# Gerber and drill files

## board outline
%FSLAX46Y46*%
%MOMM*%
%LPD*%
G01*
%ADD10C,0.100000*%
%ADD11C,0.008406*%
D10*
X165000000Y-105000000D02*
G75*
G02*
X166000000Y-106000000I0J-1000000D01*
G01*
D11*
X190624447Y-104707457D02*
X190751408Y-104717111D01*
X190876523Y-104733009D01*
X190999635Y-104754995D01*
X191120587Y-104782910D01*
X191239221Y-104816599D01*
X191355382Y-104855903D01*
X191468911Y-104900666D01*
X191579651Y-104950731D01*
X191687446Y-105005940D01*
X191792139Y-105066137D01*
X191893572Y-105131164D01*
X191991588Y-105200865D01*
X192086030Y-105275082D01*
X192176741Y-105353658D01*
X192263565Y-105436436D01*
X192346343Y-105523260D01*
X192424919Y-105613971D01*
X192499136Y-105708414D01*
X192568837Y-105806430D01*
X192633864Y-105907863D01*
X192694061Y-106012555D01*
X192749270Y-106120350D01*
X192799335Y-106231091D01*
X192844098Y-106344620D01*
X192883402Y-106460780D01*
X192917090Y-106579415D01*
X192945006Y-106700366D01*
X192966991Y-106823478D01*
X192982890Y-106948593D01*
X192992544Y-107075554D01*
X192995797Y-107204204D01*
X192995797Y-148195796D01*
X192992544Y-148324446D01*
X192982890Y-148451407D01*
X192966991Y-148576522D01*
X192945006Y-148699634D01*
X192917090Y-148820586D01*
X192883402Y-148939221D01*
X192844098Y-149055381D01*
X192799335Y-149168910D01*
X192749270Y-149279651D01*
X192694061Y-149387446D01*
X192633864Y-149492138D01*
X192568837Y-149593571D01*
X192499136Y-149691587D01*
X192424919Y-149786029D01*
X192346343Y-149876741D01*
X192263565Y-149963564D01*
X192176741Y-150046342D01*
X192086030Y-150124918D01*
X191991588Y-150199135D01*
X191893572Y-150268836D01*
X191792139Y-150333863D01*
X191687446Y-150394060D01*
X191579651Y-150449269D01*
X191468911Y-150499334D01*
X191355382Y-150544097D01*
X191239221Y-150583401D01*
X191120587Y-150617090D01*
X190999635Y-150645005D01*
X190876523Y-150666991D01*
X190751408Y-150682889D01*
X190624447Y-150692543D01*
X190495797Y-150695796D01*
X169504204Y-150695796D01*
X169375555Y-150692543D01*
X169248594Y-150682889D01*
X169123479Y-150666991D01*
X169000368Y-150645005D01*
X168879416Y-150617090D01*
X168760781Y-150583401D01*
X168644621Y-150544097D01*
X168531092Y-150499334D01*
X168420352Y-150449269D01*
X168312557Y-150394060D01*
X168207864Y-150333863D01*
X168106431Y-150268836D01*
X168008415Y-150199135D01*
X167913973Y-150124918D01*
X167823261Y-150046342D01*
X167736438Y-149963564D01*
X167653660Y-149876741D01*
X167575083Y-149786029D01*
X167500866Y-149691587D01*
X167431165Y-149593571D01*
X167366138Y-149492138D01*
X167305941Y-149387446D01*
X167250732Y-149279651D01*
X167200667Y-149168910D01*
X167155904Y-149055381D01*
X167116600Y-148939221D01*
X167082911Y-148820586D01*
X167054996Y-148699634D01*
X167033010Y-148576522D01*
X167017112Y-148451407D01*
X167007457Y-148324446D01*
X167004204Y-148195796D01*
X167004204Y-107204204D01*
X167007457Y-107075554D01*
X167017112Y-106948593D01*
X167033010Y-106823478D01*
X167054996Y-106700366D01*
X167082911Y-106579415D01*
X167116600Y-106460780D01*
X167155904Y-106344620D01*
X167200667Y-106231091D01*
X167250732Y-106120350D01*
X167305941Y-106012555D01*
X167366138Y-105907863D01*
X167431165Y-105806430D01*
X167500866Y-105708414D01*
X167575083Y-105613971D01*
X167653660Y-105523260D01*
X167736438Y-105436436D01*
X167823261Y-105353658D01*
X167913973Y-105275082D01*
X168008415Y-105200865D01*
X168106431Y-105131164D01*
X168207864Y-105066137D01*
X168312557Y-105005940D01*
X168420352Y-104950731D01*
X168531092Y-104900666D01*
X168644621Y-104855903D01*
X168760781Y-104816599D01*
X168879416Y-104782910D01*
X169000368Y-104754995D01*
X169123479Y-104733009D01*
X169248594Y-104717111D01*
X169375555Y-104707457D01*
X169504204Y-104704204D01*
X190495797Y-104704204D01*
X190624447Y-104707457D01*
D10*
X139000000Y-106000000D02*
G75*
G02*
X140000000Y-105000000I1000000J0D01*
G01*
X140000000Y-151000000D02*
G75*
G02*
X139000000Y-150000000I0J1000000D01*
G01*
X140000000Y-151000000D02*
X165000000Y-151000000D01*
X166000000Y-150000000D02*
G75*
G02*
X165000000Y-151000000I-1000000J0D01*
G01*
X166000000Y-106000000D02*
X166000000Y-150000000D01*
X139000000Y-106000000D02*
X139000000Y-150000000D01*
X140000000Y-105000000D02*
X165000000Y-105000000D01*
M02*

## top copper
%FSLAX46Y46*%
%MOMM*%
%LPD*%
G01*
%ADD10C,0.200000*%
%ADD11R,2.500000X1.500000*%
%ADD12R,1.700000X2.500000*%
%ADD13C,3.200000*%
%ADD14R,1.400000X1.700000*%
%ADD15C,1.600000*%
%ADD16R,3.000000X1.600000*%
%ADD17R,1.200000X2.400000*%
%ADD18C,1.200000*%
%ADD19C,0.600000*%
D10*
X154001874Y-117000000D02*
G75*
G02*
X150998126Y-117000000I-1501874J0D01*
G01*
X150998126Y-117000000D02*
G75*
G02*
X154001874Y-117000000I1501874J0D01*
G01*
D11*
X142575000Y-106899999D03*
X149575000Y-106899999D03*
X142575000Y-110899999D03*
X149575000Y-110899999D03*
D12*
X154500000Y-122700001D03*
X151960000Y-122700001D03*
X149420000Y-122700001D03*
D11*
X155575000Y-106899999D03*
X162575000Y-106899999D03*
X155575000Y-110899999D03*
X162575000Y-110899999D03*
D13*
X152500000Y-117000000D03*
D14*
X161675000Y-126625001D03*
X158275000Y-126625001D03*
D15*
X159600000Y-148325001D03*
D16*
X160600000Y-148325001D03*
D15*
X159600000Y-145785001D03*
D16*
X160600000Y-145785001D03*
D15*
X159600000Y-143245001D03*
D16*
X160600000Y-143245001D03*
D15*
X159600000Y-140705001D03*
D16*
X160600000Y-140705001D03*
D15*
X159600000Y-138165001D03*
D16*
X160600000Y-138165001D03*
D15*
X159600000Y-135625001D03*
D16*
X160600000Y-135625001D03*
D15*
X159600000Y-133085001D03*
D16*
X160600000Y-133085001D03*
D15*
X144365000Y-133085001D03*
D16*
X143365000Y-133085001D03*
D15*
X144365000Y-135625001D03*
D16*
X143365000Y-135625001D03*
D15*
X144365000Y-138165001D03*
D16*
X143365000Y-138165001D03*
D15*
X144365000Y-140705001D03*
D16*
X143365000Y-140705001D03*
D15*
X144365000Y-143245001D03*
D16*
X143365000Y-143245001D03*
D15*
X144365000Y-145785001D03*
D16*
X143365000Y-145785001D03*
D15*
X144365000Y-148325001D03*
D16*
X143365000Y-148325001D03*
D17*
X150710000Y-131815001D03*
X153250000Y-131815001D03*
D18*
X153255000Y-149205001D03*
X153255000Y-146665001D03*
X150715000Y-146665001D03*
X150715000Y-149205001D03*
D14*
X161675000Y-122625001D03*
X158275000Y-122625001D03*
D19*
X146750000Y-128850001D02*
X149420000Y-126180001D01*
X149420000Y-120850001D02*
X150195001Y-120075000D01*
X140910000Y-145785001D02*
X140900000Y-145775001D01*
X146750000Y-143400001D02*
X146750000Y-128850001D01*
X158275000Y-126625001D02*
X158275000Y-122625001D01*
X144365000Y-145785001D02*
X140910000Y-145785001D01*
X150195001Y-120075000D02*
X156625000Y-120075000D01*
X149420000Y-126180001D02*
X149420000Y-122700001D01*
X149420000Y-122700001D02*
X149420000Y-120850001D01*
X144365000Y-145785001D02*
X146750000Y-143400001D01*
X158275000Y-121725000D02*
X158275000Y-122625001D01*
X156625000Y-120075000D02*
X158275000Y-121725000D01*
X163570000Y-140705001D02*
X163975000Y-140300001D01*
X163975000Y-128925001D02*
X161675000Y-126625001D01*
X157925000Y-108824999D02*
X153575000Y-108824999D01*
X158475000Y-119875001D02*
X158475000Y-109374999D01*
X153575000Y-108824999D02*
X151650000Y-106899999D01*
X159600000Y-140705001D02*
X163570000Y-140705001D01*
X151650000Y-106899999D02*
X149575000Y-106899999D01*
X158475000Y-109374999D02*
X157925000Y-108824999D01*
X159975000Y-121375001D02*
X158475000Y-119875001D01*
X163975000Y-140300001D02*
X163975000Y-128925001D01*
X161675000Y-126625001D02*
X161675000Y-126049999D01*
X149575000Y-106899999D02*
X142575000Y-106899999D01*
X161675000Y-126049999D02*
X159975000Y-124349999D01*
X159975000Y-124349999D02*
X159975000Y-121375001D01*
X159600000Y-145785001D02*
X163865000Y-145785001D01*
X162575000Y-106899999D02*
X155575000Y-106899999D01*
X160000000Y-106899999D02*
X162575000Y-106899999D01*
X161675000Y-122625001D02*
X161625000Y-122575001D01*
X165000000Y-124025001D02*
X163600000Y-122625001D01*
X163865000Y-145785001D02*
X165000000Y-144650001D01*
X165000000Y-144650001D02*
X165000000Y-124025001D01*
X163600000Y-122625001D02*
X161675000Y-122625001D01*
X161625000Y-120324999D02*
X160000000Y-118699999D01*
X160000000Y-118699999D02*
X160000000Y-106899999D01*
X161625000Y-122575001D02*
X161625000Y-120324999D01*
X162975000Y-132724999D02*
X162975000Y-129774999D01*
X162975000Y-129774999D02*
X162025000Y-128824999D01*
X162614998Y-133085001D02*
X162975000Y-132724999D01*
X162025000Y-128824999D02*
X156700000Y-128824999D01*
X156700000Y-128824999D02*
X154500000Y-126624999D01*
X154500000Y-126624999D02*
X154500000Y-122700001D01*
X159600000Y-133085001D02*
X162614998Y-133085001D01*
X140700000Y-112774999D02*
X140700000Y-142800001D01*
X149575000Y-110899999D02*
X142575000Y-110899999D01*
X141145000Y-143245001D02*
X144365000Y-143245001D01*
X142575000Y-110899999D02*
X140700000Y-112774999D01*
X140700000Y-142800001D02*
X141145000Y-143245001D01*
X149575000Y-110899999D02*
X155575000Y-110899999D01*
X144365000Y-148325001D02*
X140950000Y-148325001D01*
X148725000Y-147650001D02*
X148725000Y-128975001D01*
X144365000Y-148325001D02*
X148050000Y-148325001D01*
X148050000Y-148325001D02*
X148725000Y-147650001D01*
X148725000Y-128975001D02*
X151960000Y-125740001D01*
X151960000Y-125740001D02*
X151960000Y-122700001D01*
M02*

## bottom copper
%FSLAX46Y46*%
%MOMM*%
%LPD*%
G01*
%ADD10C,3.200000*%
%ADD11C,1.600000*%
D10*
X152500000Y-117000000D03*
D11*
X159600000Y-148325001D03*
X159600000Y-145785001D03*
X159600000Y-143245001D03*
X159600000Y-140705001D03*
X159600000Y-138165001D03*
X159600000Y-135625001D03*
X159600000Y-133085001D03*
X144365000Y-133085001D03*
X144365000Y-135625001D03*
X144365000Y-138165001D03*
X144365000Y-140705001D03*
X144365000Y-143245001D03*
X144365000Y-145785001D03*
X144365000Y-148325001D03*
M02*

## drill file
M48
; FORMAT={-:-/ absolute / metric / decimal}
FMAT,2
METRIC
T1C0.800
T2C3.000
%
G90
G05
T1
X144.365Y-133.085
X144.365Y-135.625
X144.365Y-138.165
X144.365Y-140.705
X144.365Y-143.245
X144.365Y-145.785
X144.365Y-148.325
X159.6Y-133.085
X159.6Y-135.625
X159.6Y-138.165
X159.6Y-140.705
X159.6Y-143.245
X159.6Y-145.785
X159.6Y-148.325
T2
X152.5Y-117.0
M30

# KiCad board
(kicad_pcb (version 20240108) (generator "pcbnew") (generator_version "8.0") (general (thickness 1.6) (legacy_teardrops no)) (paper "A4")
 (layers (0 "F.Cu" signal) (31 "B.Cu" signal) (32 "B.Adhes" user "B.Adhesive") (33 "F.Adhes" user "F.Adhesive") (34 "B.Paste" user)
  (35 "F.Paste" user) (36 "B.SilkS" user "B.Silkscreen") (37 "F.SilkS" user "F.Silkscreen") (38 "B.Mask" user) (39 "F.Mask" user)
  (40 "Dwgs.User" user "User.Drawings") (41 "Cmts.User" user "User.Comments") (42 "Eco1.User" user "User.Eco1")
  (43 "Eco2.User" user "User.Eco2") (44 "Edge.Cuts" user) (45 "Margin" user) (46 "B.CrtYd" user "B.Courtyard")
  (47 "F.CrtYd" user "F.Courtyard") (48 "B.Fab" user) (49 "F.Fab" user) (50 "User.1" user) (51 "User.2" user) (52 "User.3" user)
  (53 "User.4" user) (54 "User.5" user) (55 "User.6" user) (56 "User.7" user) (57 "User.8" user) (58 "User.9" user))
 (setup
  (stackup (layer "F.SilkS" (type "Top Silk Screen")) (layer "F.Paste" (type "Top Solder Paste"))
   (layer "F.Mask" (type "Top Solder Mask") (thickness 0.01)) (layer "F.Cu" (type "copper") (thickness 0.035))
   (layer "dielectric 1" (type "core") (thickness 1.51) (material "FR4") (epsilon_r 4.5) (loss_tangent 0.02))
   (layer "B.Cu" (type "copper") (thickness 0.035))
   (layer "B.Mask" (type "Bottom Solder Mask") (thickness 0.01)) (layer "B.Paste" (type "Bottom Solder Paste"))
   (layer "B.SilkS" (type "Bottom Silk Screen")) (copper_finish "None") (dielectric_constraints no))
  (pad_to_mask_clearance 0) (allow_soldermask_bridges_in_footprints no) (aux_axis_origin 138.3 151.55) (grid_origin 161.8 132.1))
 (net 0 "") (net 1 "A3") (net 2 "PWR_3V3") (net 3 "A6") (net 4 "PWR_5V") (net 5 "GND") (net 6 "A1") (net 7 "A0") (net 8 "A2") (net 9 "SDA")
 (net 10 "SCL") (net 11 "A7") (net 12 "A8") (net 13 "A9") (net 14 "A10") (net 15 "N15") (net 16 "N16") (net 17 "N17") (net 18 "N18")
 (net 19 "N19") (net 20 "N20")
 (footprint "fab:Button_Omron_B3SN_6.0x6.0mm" (layer "F.Cu") (at 146.075 108.899999)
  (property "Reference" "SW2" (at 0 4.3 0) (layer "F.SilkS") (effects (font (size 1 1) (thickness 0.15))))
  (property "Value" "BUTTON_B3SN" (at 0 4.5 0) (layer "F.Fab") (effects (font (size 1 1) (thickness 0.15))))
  (pad "1" smd rect (at -3.5 -2) (size 2.5 1.5) (layers "F.Cu" "F.Paste" "F.Mask") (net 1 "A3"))
  (pad "1" smd rect (at 3.5 -2) (size 2.5 1.5) (layers "F.Cu" "F.Paste" "F.Mask") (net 1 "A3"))
  (pad "2" smd rect (at -3.5 2) (size 2.5 1.5) (layers "F.Cu" "F.Paste" "F.Mask") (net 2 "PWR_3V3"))
  (pad "2" smd rect (at 3.5 2) (size 2.5 1.5) (layers "F.Cu" "F.Paste" "F.Mask") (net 2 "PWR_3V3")))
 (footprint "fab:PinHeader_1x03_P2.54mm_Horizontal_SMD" (layer "F.Cu") (at 154.5 122.700001 -90)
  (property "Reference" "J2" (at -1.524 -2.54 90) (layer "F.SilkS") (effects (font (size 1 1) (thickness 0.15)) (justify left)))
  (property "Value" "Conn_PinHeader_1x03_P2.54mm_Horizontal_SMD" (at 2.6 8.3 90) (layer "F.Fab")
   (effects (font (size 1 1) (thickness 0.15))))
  (pad "1" smd rect (at 0 0 270) (size 2.5 1.7) (layers "F.Cu" "F.Paste" "F.Mask") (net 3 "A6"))
  (pad "2" smd rect (at 0 2.54 270) (size 2.5 1.7) (layers "F.Cu" "F.Paste" "F.Mask") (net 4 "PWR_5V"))
  (pad "3" smd rect (at 0 5.08 270) (size 2.5 1.7) (layers "F.Cu" "F.Paste" "F.Mask") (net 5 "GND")))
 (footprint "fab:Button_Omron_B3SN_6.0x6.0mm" (layer "F.Cu") (at 159.075 108.899999)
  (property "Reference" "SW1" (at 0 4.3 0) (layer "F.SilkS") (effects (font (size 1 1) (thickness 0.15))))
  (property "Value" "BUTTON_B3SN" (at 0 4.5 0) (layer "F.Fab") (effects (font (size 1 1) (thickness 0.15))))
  (pad "1" smd rect (at -3.5 -2) (size 2.5 1.5) (layers "F.Cu" "F.Paste" "F.Mask") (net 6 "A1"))
  (pad "1" smd rect (at 3.5 -2) (size 2.5 1.5) (layers "F.Cu" "F.Paste" "F.Mask") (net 6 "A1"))
  (pad "2" smd rect (at -3.5 2) (size 2.5 1.5) (layers "F.Cu" "F.Paste" "F.Mask") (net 2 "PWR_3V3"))
  (pad "2" smd rect (at 3.5 2) (size 2.5 1.5) (layers "F.Cu" "F.Paste" "F.Mask") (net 2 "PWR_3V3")))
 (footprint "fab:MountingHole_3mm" (layer "F.Cu") (at 152.5 117)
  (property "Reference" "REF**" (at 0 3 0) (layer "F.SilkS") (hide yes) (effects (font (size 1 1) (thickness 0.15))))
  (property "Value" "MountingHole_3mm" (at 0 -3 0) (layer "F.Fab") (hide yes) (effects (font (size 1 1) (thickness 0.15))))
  (pad "" thru_hole circle (at 0 0) (size 3.2 3.2) (drill 3) (layers "*.Cu" "*.Mask") (remove_unused_layers no)))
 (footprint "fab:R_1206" (layer "F.Cu") (at 159.975 126.625001 180)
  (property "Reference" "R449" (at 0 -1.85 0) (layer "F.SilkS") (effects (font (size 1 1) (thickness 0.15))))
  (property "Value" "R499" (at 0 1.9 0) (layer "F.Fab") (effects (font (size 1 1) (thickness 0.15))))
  (pad "1" smd rect (at -1.7 0 180) (size 1.4 1.7) (layers "F.Cu" "F.Paste" "F.Mask") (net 1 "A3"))
  (pad "2" smd rect (at 1.7 0 180) (size 1.4 1.7) (layers "F.Cu" "F.Paste" "F.Mask") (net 5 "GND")))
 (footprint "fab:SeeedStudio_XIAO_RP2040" (layer "F.Cu") (at 151.985 140.705001 180)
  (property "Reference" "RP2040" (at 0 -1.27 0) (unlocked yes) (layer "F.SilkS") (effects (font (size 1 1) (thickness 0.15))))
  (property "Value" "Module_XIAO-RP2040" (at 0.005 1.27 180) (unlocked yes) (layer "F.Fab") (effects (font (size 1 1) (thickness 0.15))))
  (pad "1" thru_hole circle (at -7.615 -7.62 180) (size 1.6 1.6) (drill 0.8) (layers "*.Cu" "*.Mask") (remove_unused_layers no) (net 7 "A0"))
  (pad "1" smd rect (at -7.615 -7.62 180) (size 3 1.6) (drill (offset -1 0)) (layers "F.Cu" "F.Paste" "F.Mask") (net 7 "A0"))
  (pad "2" thru_hole circle (at -7.615 -5.08 180) (size 1.6 1.6) (drill 0.8) (layers "*.Cu" "*.Mask") (remove_unused_layers no) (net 6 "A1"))
  (pad "2" smd rect (at -7.615 -5.08 180) (size 3 1.6) (drill (offset -1 0)) (layers "F.Cu" "F.Paste" "F.Mask") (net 6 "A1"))
  (pad "3" thru_hole circle (at -7.615 -2.54 180) (size 1.6 1.6) (drill 0.8) (layers "*.Cu" "*.Mask") (remove_unused_layers no) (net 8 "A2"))
  (pad "3" smd rect (at -7.615 -2.54 180) (size 3 1.6) (drill (offset -1 0)) (layers "F.Cu" "F.Paste" "F.Mask") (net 8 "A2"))
  (pad "4" thru_hole circle (at -7.615 0 180) (size 1.6 1.6) (drill 0.8) (layers "*.Cu" "*.Mask") (remove_unused_layers no) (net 1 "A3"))
  (pad "4" smd rect (at -7.615 0 180) (size 3 1.6) (drill (offset -1 0)) (layers "F.Cu" "F.Paste" "F.Mask") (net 1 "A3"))
  (pad "5" thru_hole circle (at -7.615 2.54 180) (size 1.6 1.6) (drill 0.8) (layers "*.Cu" "*.Mask") (remove_unused_layers no) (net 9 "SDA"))
  (pad "5" smd rect (at -7.615 2.54 180) (size 3 1.6) (drill (offset -1 0)) (layers "F.Cu" "F.Paste" "F.Mask") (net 9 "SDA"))
  (pad "6" thru_hole circle (at -7.615 5.08 180) (size 1.6 1.6) (drill 0.8) (layers "*.Cu" "*.Mask") (remove_unused_layers no)
   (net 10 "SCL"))
  (pad "6" smd rect (at -7.615 5.08 180) (size 3 1.6) (drill (offset -1 0)) (layers "F.Cu" "F.Paste" "F.Mask") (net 10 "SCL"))
  (pad "7" thru_hole circle (at -7.615 7.62 180) (size 1.6 1.6) (drill 0.8) (layers "*.Cu" "*.Mask") (remove_unused_layers no) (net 3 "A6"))
  (pad "7" smd rect (at -7.615 7.62 180) (size 3 1.6) (drill (offset -1 0)) (layers "F.Cu" "F.Paste" "F.Mask") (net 3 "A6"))
  (pad "8" thru_hole circle (at 7.62 7.62 180) (size 1.6 1.6) (drill 0.8) (layers "*.Cu" "*.Mask") (remove_unused_layers no) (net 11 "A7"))
  (pad "8" smd rect (at 7.62 7.62 180) (size 3 1.6) (drill (offset 1 0)) (layers "F.Cu" "F.Paste" "F.Mask") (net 11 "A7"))
  (pad "9" thru_hole circle (at 7.62 5.08 180) (size 1.6 1.6) (drill 0.8) (layers "*.Cu" "*.Mask") (remove_unused_layers no) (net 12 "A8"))
  (pad "9" smd rect (at 7.62 5.08 180) (size 3 1.6) (drill (offset 1 0)) (layers "F.Cu" "F.Paste" "F.Mask") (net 12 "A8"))
  (pad "10" thru_hole circle (at 7.62 2.54 180) (size 1.6 1.6) (drill 0.8) (layers "*.Cu" "*.Mask") (remove_unused_layers no) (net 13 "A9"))
  (pad "10" smd rect (at 7.62 2.54 180) (size 3 1.6) (drill (offset 1 0)) (layers "F.Cu" "F.Paste" "F.Mask") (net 13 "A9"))
  (pad "11" thru_hole circle (at 7.62 0 180) (size 1.6 1.6) (drill 0.8) (layers "*.Cu" "*.Mask") (remove_unused_layers no) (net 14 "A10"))
  (pad "11" smd rect (at 7.62 0 180) (size 3 1.6) (drill (offset 1 0)) (layers "F.Cu" "F.Paste" "F.Mask") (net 14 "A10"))
  (pad "12" thru_hole circle (at 7.62 -2.54 180) (size 1.6 1.6) (drill 0.8) (layers "*.Cu" "*.Mask") (remove_unused_layers no)
   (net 2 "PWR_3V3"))
  (pad "12" smd rect (at 7.62 -2.54 180) (size 3 1.6) (drill (offset 1 0)) (layers "F.Cu" "F.Paste" "F.Mask") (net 2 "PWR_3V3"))
  (pad "13" thru_hole circle (at 7.62 -5.08 180) (size 1.6 1.6) (drill 0.8) (layers "*.Cu" "*.Mask") (remove_unused_layers no) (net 5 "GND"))
  (pad "13" smd rect (at 7.62 -5.08 180) (size 3 1.6) (drill (offset 1 0)) (layers "F.Cu" "F.Paste" "F.Mask") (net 5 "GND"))
  (pad "14" thru_hole circle (at 7.62 -7.62 180) (size 1.6 1.6) (drill 0.8) (layers "*.Cu" "*.Mask") (remove_unused_layers no)
   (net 4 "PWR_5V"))
  (pad "14" smd rect (at 7.62 -7.62 180) (size 3 1.6) (drill (offset 1 0)) (layers "F.Cu" "F.Paste" "F.Mask") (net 4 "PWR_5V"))
  (pad "15" smd rect (at 1.275 8.89 90) (size 2.4 1.2) (layers "F.Cu" "F.Paste" "F.Mask") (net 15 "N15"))
  (pad "16" smd rect (at -1.265 8.89 90) (size 2.4 1.2) (layers "F.Cu" "F.Paste" "F.Mask") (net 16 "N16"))
  (pad "17" smd circle (at -1.27 -8.5 180) (size 1.2 1.2) (layers "F.Cu" "F.Paste" "F.Mask") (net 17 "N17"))
  (pad "18" smd circle (at -1.27 -5.96 180) (size 1.2 1.2) (layers "F.Cu" "F.Paste" "F.Mask") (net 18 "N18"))
  (pad "19" smd circle (at 1.27 -5.96 180) (size 1.2 1.2) (layers "F.Cu" "F.Paste" "F.Mask") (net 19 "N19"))
  (pad "20" smd circle (at 1.27 -8.5 180) (size 1.2 1.2) (layers "F.Cu" "F.Paste" "F.Mask") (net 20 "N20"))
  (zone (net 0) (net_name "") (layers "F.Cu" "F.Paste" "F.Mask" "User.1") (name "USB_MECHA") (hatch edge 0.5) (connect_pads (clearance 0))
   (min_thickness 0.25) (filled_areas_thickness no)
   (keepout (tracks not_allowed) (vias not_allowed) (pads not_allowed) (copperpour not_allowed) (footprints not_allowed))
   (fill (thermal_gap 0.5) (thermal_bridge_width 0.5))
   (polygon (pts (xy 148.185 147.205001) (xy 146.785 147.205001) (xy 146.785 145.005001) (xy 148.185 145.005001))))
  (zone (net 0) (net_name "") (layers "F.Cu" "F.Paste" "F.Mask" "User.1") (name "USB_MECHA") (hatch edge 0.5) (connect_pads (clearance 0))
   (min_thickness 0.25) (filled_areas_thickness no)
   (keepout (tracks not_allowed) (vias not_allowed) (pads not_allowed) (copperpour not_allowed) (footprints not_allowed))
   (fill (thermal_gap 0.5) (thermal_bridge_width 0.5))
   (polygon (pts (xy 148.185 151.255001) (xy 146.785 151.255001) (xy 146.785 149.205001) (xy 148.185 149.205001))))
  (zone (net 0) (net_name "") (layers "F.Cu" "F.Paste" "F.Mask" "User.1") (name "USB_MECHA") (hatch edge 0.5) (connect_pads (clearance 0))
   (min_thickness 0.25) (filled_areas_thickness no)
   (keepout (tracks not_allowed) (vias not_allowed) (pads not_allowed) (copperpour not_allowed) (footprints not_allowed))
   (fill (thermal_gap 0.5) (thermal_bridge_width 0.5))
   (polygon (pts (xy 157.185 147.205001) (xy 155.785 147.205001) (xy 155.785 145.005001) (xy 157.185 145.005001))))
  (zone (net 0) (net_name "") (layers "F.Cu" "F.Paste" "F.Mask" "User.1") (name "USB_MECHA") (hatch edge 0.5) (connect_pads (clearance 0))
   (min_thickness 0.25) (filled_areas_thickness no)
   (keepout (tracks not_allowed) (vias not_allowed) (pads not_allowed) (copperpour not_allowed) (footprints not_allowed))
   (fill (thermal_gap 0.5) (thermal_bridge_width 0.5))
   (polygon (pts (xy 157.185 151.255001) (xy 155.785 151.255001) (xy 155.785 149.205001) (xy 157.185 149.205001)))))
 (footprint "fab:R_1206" (layer "F.Cu") (at 159.975 122.625001 180)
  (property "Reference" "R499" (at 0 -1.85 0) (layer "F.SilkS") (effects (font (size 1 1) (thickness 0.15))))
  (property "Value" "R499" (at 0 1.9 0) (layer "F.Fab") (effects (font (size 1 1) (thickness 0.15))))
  (pad "1" smd rect (at -1.7 0 180) (size 1.4 1.7) (layers "F.Cu" "F.Paste" "F.Mask") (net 6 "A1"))
  (pad "2" smd rect (at 1.7 0 180) (size 1.4 1.7) (layers "F.Cu" "F.Paste" "F.Mask") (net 5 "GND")))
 (gr_circle (center 152.5 117) (end 154 116.925) (stroke (width 0.2) (type default)) (fill none) (layer "F.Cu"))
 (gr_arc (start 165 105) (mid 165.707106 105.292894) (end 166 106) (stroke (width 0.1) (type default)) (layer "Edge.Cuts"))
 (gr_poly
  (pts (xy 190.624447 104.707457) (xy 190.751408 104.717111) (xy 190.876523 104.733009) (xy 190.999635 104.754995) (xy 191.120587 104.78291)
   (xy 191.239221 104.816599) (xy 191.355382 104.855903) (xy 191.468911 104.900666) (xy 191.579651 104.950731) (xy 191.687446 105.00594)
   (xy 191.792139 105.066137) (xy 191.893572 105.131164) (xy 191.991588 105.200865) (xy 192.08603 105.275082) (xy 192.176741 105.353658)
   (xy 192.263565 105.436436) (xy 192.346343 105.52326) (xy 192.424919 105.613971) (xy 192.499136 105.708414) (xy 192.568837 105.80643)
   (xy 192.633864 105.907863) (xy 192.694061 106.012555) (xy 192.74927 106.12035) (xy 192.799335 106.231091) (xy 192.844098 106.34462)
   (xy 192.883402 106.46078) (xy 192.91709 106.579415) (xy 192.945006 106.700366) (xy 192.966991 106.823478) (xy 192.98289 106.948593)
   (xy 192.992544 107.075554) (xy 192.995797 107.204204) (xy 192.995797 148.195796) (xy 192.992544 148.324446) (xy 192.98289 148.451407)
   (xy 192.966991 148.576522) (xy 192.945006 148.699634) (xy 192.91709 148.820586) (xy 192.883402 148.939221) (xy 192.844098 149.055381)
   (xy 192.799335 149.16891) (xy 192.74927 149.279651) (xy 192.694061 149.387446) (xy 192.633864 149.492138) (xy 192.568837 149.593571)
   (xy 192.499136 149.691587) (xy 192.424919 149.786029) (xy 192.346343 149.876741) (xy 192.263565 149.963564) (xy 192.176741 150.046342)
   (xy 192.08603 150.124918) (xy 191.991588 150.199135) (xy 191.893572 150.268836) (xy 191.792139 150.333863) (xy 191.687446 150.39406)
   (xy 191.579651 150.449269) (xy 191.468911 150.499334) (xy 191.355382 150.544097) (xy 191.239221 150.583401) (xy 191.120587 150.61709)
   (xy 190.999635 150.645005) (xy 190.876523 150.666991) (xy 190.751408 150.682889) (xy 190.624447 150.692543) (xy 190.495797 150.695796)
   (xy 169.504204 150.695796) (xy 169.375555 150.692543) (xy 169.248594 150.682889) (xy 169.123479 150.666991) (xy 169.000368 150.645005)
   (xy 168.879416 150.61709) (xy 168.760781 150.583401) (xy 168.644621 150.544097) (xy 168.531092 150.499334) (xy 168.420352 150.449269)
   (xy 168.312557 150.39406) (xy 168.207864 150.333863) (xy 168.106431 150.268836) (xy 168.008415 150.199135) (xy 167.913973 150.124918)
   (xy 167.823261 150.046342) (xy 167.736438 149.963564) (xy 167.65366 149.876741) (xy 167.575083 149.786029) (xy 167.500866 149.691587)
   (xy 167.431165 149.593571) (xy 167.366138 149.492138) (xy 167.305941 149.387446) (xy 167.250732 149.279651) (xy 167.200667 149.16891)
   (xy 167.155904 149.055381) (xy 167.1166 148.939221) (xy 167.082911 148.820586) (xy 167.054996 148.699634) (xy 167.03301 148.576522)
   (xy 167.017112 148.451407) (xy 167.007457 148.324446) (xy 167.004204 148.195796) (xy 167.004204 107.204204) (xy 167.007457 107.075554)
   (xy 167.017112 106.948593) (xy 167.03301 106.823478) (xy 167.054996 106.700366) (xy 167.082911 106.579415) (xy 167.1166 106.46078)
   (xy 167.155904 106.34462) (xy 167.200667 106.231091) (xy 167.250732 106.12035) (xy 167.305941 106.012555) (xy 167.366138 105.907863)
   (xy 167.431165 105.80643) (xy 167.500866 105.708414) (xy 167.575083 105.613971) (xy 167.65366 105.52326) (xy 167.736438 105.436436)
   (xy 167.823261 105.353658) (xy 167.913973 105.275082) (xy 168.008415 105.200865) (xy 168.106431 105.131164) (xy 168.207864 105.066137)
   (xy 168.312557 105.00594) (xy 168.420352 104.950731) (xy 168.531092 104.900666) (xy 168.644621 104.855903) (xy 168.760781 104.816599)
   (xy 168.879416 104.78291) (xy 169.000368 104.754995) (xy 169.123479 104.733009) (xy 169.248594 104.717111) (xy 169.375555 104.707457)
   (xy 169.504204 104.704204) (xy 190.495797 104.704204))
  (stroke (width 0.008406) (type solid)) (fill none) (layer "Edge.Cuts"))
 (gr_arc (start 139 106) (mid 139.292893 105.292894) (end 140 105) (stroke (width 0.1) (type default)) (layer "Edge.Cuts"))
 (gr_arc (start 140 151) (mid 139.292895 150.707106) (end 139 150) (stroke (width 0.1) (type default)) (layer "Edge.Cuts"))
 (gr_line (start 140 151) (end 165 151) (stroke (width 0.1) (type default)) (layer "Edge.Cuts"))
 (gr_arc (start 166 150) (mid 165.707106 150.707105) (end 165 151) (stroke (width 0.1) (type default)) (layer "Edge.Cuts"))
 (gr_line (start 166 106) (end 166 150) (stroke (width 0.1) (type default)) (layer "Edge.Cuts"))
 (gr_line (start 139 106) (end 139 150) (stroke (width 0.1) (type default)) (layer "Edge.Cuts"))
 (gr_line (start 140 105) (end 165 105) (stroke (width 0.1) (type default)) (layer "Edge.Cuts"))
 (segment (start 146.75 128.850001) (end 149.42 126.180001) (width 0.6) (layer "F.Cu") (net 5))
 (segment (start 149.42 120.850001) (end 150.195001 120.075) (width 0.6) (layer "F.Cu") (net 5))
 (segment (start 140.91 145.785001) (end 140.9 145.775001) (width 0.6) (layer "F.Cu") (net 5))
 (segment (start 146.75 143.400001) (end 146.75 128.850001) (width 0.6) (layer "F.Cu") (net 5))
 (segment (start 158.275 126.625001) (end 158.275 122.625001) (width 0.6) (layer "F.Cu") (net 5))
 (segment (start 144.365 145.785001) (end 140.91 145.785001) (width 0.6) (layer "F.Cu") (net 5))
 (segment (start 150.195001 120.075) (end 156.625 120.075) (width 0.6) (layer "F.Cu") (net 5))
 (segment (start 149.42 126.180001) (end 149.42 122.700001) (width 0.6) (layer "F.Cu") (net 5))
 (segment (start 149.42 122.700001) (end 149.42 120.850001) (width 0.6) (layer "F.Cu") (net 5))
 (segment (start 144.365 145.785001) (end 146.75 143.400001) (width 0.6) (layer "F.Cu") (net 5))
 (segment (start 158.275 121.725) (end 158.275 122.625001) (width 0.6) (layer "F.Cu") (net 5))
 (segment (start 156.625 120.075) (end 158.275 121.725) (width 0.6) (layer "F.Cu") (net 5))
 (segment (start 163.57 140.705001) (end 163.975 140.300001) (width 0.6) (layer "F.Cu") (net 1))
 (segment (start 163.975 128.925001) (end 161.675 126.625001) (width 0.6) (layer "F.Cu") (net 1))
 (segment (start 157.925 108.824999) (end 153.575 108.824999) (width 0.6) (layer "F.Cu") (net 1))
 (segment (start 158.475 119.875001) (end 158.475 109.374999) (width 0.6) (layer "F.Cu") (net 1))
 (segment (start 153.575 108.824999) (end 151.65 106.899999) (width 0.6) (layer "F.Cu") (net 1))
 (segment (start 159.6 140.705001) (end 163.57 140.705001) (width 0.6) (layer "F.Cu") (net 1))
 (segment (start 151.65 106.899999) (end 149.575 106.899999) (width 0.6) (layer "F.Cu") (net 1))
 (segment (start 158.475 109.374999) (end 157.925 108.824999) (width 0.6) (layer "F.Cu") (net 1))
 (segment (start 159.975 121.375001) (end 158.475 119.875001) (width 0.6) (layer "F.Cu") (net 1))
 (segment (start 163.975 140.300001) (end 163.975 128.925001) (width 0.6) (layer "F.Cu") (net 1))
 (segment (start 161.675 126.625001) (end 161.675 126.049999) (width 0.6) (layer "F.Cu") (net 1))
 (segment (start 149.575 106.899999) (end 142.575 106.899999) (width 0.6) (layer "F.Cu") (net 1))
 (segment (start 161.675 126.049999) (end 159.975 124.349999) (width 0.6) (layer "F.Cu") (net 1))
 (segment (start 159.975 124.349999) (end 159.975 121.375001) (width 0.6) (layer "F.Cu") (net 1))
 (segment (start 159.6 145.785001) (end 163.865 145.785001) (width 0.6) (layer "F.Cu") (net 6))
 (segment (start 162.575 106.899999) (end 155.575 106.899999) (width 0.6) (layer "F.Cu") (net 6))
 (segment (start 160 106.899999) (end 162.575 106.899999) (width 0.6) (layer "F.Cu") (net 6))
 (segment (start 161.675 122.625001) (end 161.625 122.575001) (width 0.6) (layer "F.Cu") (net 6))
 (segment (start 165 124.025001) (end 163.6 122.625001) (width 0.6) (layer "F.Cu") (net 6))
 (segment (start 163.865 145.785001) (end 165 144.650001) (width 0.6) (layer "F.Cu") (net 6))
 (segment (start 165 144.650001) (end 165 124.025001) (width 0.6) (layer "F.Cu") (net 6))
 (segment (start 163.6 122.625001) (end 161.675 122.625001) (width 0.6) (layer "F.Cu") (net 6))
 (segment (start 161.625 120.324999) (end 160 118.699999) (width 0.6) (layer "F.Cu") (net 6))
 (segment (start 160 118.699999) (end 160 106.899999) (width 0.6) (layer "F.Cu") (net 6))
 (segment (start 161.625 122.575001) (end 161.625 120.324999) (width 0.6) (layer "F.Cu") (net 6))
 (segment (start 162.975 132.724999) (end 162.975 129.774999) (width 0.6) (layer "F.Cu") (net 3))
 (segment (start 162.975 129.774999) (end 162.025 128.824999) (width 0.6) (layer "F.Cu") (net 3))
 (segment (start 162.614998 133.085001) (end 162.975 132.724999) (width 0.6) (layer "F.Cu") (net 3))
 (segment (start 162.025 128.824999) (end 156.7 128.824999) (width 0.6) (layer "F.Cu") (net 3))
 (segment (start 156.7 128.824999) (end 154.5 126.624999) (width 0.6) (layer "F.Cu") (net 3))
 (segment (start 154.5 126.624999) (end 154.5 122.700001) (width 0.6) (layer "F.Cu") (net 3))
 (segment (start 159.6 133.085001) (end 162.614998 133.085001) (width 0.6) (layer "F.Cu") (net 3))
 (segment (start 140.7 112.774999) (end 140.7 142.800001) (width 0.6) (layer "F.Cu") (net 2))
 (segment (start 149.575 110.899999) (end 142.575 110.899999) (width 0.6) (layer "F.Cu") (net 2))
 (segment (start 141.145 143.245001) (end 144.365 143.245001) (width 0.6) (layer "F.Cu") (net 2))
 (segment (start 142.575 110.899999) (end 140.7 112.774999) (width 0.6) (layer "F.Cu") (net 2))
 (segment (start 140.7 142.800001) (end 141.145 143.245001) (width 0.6) (layer "F.Cu") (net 2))
 (segment (start 149.575 110.899999) (end 155.575 110.899999) (width 0.6) (layer "F.Cu") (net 2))
 (segment (start 144.365 148.325001) (end 140.95 148.325001) (width 0.6) (layer "F.Cu") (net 4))
 (segment (start 148.725 147.650001) (end 148.725 128.975001) (width 0.6) (layer "F.Cu") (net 4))
 (segment (start 144.365 148.325001) (end 148.05 148.325001) (width 0.6) (layer "F.Cu") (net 4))
 (segment (start 148.05 148.325001) (end 148.725 147.650001) (width 0.6) (layer "F.Cu") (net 4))
 (segment (start 148.725 128.975001) (end 151.96 125.740001) (width 0.6) (layer "F.Cu") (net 4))
 (segment (start 151.96 125.740001) (end 151.96 122.700001) (width 0.6) (layer "F.Cu") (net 4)))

